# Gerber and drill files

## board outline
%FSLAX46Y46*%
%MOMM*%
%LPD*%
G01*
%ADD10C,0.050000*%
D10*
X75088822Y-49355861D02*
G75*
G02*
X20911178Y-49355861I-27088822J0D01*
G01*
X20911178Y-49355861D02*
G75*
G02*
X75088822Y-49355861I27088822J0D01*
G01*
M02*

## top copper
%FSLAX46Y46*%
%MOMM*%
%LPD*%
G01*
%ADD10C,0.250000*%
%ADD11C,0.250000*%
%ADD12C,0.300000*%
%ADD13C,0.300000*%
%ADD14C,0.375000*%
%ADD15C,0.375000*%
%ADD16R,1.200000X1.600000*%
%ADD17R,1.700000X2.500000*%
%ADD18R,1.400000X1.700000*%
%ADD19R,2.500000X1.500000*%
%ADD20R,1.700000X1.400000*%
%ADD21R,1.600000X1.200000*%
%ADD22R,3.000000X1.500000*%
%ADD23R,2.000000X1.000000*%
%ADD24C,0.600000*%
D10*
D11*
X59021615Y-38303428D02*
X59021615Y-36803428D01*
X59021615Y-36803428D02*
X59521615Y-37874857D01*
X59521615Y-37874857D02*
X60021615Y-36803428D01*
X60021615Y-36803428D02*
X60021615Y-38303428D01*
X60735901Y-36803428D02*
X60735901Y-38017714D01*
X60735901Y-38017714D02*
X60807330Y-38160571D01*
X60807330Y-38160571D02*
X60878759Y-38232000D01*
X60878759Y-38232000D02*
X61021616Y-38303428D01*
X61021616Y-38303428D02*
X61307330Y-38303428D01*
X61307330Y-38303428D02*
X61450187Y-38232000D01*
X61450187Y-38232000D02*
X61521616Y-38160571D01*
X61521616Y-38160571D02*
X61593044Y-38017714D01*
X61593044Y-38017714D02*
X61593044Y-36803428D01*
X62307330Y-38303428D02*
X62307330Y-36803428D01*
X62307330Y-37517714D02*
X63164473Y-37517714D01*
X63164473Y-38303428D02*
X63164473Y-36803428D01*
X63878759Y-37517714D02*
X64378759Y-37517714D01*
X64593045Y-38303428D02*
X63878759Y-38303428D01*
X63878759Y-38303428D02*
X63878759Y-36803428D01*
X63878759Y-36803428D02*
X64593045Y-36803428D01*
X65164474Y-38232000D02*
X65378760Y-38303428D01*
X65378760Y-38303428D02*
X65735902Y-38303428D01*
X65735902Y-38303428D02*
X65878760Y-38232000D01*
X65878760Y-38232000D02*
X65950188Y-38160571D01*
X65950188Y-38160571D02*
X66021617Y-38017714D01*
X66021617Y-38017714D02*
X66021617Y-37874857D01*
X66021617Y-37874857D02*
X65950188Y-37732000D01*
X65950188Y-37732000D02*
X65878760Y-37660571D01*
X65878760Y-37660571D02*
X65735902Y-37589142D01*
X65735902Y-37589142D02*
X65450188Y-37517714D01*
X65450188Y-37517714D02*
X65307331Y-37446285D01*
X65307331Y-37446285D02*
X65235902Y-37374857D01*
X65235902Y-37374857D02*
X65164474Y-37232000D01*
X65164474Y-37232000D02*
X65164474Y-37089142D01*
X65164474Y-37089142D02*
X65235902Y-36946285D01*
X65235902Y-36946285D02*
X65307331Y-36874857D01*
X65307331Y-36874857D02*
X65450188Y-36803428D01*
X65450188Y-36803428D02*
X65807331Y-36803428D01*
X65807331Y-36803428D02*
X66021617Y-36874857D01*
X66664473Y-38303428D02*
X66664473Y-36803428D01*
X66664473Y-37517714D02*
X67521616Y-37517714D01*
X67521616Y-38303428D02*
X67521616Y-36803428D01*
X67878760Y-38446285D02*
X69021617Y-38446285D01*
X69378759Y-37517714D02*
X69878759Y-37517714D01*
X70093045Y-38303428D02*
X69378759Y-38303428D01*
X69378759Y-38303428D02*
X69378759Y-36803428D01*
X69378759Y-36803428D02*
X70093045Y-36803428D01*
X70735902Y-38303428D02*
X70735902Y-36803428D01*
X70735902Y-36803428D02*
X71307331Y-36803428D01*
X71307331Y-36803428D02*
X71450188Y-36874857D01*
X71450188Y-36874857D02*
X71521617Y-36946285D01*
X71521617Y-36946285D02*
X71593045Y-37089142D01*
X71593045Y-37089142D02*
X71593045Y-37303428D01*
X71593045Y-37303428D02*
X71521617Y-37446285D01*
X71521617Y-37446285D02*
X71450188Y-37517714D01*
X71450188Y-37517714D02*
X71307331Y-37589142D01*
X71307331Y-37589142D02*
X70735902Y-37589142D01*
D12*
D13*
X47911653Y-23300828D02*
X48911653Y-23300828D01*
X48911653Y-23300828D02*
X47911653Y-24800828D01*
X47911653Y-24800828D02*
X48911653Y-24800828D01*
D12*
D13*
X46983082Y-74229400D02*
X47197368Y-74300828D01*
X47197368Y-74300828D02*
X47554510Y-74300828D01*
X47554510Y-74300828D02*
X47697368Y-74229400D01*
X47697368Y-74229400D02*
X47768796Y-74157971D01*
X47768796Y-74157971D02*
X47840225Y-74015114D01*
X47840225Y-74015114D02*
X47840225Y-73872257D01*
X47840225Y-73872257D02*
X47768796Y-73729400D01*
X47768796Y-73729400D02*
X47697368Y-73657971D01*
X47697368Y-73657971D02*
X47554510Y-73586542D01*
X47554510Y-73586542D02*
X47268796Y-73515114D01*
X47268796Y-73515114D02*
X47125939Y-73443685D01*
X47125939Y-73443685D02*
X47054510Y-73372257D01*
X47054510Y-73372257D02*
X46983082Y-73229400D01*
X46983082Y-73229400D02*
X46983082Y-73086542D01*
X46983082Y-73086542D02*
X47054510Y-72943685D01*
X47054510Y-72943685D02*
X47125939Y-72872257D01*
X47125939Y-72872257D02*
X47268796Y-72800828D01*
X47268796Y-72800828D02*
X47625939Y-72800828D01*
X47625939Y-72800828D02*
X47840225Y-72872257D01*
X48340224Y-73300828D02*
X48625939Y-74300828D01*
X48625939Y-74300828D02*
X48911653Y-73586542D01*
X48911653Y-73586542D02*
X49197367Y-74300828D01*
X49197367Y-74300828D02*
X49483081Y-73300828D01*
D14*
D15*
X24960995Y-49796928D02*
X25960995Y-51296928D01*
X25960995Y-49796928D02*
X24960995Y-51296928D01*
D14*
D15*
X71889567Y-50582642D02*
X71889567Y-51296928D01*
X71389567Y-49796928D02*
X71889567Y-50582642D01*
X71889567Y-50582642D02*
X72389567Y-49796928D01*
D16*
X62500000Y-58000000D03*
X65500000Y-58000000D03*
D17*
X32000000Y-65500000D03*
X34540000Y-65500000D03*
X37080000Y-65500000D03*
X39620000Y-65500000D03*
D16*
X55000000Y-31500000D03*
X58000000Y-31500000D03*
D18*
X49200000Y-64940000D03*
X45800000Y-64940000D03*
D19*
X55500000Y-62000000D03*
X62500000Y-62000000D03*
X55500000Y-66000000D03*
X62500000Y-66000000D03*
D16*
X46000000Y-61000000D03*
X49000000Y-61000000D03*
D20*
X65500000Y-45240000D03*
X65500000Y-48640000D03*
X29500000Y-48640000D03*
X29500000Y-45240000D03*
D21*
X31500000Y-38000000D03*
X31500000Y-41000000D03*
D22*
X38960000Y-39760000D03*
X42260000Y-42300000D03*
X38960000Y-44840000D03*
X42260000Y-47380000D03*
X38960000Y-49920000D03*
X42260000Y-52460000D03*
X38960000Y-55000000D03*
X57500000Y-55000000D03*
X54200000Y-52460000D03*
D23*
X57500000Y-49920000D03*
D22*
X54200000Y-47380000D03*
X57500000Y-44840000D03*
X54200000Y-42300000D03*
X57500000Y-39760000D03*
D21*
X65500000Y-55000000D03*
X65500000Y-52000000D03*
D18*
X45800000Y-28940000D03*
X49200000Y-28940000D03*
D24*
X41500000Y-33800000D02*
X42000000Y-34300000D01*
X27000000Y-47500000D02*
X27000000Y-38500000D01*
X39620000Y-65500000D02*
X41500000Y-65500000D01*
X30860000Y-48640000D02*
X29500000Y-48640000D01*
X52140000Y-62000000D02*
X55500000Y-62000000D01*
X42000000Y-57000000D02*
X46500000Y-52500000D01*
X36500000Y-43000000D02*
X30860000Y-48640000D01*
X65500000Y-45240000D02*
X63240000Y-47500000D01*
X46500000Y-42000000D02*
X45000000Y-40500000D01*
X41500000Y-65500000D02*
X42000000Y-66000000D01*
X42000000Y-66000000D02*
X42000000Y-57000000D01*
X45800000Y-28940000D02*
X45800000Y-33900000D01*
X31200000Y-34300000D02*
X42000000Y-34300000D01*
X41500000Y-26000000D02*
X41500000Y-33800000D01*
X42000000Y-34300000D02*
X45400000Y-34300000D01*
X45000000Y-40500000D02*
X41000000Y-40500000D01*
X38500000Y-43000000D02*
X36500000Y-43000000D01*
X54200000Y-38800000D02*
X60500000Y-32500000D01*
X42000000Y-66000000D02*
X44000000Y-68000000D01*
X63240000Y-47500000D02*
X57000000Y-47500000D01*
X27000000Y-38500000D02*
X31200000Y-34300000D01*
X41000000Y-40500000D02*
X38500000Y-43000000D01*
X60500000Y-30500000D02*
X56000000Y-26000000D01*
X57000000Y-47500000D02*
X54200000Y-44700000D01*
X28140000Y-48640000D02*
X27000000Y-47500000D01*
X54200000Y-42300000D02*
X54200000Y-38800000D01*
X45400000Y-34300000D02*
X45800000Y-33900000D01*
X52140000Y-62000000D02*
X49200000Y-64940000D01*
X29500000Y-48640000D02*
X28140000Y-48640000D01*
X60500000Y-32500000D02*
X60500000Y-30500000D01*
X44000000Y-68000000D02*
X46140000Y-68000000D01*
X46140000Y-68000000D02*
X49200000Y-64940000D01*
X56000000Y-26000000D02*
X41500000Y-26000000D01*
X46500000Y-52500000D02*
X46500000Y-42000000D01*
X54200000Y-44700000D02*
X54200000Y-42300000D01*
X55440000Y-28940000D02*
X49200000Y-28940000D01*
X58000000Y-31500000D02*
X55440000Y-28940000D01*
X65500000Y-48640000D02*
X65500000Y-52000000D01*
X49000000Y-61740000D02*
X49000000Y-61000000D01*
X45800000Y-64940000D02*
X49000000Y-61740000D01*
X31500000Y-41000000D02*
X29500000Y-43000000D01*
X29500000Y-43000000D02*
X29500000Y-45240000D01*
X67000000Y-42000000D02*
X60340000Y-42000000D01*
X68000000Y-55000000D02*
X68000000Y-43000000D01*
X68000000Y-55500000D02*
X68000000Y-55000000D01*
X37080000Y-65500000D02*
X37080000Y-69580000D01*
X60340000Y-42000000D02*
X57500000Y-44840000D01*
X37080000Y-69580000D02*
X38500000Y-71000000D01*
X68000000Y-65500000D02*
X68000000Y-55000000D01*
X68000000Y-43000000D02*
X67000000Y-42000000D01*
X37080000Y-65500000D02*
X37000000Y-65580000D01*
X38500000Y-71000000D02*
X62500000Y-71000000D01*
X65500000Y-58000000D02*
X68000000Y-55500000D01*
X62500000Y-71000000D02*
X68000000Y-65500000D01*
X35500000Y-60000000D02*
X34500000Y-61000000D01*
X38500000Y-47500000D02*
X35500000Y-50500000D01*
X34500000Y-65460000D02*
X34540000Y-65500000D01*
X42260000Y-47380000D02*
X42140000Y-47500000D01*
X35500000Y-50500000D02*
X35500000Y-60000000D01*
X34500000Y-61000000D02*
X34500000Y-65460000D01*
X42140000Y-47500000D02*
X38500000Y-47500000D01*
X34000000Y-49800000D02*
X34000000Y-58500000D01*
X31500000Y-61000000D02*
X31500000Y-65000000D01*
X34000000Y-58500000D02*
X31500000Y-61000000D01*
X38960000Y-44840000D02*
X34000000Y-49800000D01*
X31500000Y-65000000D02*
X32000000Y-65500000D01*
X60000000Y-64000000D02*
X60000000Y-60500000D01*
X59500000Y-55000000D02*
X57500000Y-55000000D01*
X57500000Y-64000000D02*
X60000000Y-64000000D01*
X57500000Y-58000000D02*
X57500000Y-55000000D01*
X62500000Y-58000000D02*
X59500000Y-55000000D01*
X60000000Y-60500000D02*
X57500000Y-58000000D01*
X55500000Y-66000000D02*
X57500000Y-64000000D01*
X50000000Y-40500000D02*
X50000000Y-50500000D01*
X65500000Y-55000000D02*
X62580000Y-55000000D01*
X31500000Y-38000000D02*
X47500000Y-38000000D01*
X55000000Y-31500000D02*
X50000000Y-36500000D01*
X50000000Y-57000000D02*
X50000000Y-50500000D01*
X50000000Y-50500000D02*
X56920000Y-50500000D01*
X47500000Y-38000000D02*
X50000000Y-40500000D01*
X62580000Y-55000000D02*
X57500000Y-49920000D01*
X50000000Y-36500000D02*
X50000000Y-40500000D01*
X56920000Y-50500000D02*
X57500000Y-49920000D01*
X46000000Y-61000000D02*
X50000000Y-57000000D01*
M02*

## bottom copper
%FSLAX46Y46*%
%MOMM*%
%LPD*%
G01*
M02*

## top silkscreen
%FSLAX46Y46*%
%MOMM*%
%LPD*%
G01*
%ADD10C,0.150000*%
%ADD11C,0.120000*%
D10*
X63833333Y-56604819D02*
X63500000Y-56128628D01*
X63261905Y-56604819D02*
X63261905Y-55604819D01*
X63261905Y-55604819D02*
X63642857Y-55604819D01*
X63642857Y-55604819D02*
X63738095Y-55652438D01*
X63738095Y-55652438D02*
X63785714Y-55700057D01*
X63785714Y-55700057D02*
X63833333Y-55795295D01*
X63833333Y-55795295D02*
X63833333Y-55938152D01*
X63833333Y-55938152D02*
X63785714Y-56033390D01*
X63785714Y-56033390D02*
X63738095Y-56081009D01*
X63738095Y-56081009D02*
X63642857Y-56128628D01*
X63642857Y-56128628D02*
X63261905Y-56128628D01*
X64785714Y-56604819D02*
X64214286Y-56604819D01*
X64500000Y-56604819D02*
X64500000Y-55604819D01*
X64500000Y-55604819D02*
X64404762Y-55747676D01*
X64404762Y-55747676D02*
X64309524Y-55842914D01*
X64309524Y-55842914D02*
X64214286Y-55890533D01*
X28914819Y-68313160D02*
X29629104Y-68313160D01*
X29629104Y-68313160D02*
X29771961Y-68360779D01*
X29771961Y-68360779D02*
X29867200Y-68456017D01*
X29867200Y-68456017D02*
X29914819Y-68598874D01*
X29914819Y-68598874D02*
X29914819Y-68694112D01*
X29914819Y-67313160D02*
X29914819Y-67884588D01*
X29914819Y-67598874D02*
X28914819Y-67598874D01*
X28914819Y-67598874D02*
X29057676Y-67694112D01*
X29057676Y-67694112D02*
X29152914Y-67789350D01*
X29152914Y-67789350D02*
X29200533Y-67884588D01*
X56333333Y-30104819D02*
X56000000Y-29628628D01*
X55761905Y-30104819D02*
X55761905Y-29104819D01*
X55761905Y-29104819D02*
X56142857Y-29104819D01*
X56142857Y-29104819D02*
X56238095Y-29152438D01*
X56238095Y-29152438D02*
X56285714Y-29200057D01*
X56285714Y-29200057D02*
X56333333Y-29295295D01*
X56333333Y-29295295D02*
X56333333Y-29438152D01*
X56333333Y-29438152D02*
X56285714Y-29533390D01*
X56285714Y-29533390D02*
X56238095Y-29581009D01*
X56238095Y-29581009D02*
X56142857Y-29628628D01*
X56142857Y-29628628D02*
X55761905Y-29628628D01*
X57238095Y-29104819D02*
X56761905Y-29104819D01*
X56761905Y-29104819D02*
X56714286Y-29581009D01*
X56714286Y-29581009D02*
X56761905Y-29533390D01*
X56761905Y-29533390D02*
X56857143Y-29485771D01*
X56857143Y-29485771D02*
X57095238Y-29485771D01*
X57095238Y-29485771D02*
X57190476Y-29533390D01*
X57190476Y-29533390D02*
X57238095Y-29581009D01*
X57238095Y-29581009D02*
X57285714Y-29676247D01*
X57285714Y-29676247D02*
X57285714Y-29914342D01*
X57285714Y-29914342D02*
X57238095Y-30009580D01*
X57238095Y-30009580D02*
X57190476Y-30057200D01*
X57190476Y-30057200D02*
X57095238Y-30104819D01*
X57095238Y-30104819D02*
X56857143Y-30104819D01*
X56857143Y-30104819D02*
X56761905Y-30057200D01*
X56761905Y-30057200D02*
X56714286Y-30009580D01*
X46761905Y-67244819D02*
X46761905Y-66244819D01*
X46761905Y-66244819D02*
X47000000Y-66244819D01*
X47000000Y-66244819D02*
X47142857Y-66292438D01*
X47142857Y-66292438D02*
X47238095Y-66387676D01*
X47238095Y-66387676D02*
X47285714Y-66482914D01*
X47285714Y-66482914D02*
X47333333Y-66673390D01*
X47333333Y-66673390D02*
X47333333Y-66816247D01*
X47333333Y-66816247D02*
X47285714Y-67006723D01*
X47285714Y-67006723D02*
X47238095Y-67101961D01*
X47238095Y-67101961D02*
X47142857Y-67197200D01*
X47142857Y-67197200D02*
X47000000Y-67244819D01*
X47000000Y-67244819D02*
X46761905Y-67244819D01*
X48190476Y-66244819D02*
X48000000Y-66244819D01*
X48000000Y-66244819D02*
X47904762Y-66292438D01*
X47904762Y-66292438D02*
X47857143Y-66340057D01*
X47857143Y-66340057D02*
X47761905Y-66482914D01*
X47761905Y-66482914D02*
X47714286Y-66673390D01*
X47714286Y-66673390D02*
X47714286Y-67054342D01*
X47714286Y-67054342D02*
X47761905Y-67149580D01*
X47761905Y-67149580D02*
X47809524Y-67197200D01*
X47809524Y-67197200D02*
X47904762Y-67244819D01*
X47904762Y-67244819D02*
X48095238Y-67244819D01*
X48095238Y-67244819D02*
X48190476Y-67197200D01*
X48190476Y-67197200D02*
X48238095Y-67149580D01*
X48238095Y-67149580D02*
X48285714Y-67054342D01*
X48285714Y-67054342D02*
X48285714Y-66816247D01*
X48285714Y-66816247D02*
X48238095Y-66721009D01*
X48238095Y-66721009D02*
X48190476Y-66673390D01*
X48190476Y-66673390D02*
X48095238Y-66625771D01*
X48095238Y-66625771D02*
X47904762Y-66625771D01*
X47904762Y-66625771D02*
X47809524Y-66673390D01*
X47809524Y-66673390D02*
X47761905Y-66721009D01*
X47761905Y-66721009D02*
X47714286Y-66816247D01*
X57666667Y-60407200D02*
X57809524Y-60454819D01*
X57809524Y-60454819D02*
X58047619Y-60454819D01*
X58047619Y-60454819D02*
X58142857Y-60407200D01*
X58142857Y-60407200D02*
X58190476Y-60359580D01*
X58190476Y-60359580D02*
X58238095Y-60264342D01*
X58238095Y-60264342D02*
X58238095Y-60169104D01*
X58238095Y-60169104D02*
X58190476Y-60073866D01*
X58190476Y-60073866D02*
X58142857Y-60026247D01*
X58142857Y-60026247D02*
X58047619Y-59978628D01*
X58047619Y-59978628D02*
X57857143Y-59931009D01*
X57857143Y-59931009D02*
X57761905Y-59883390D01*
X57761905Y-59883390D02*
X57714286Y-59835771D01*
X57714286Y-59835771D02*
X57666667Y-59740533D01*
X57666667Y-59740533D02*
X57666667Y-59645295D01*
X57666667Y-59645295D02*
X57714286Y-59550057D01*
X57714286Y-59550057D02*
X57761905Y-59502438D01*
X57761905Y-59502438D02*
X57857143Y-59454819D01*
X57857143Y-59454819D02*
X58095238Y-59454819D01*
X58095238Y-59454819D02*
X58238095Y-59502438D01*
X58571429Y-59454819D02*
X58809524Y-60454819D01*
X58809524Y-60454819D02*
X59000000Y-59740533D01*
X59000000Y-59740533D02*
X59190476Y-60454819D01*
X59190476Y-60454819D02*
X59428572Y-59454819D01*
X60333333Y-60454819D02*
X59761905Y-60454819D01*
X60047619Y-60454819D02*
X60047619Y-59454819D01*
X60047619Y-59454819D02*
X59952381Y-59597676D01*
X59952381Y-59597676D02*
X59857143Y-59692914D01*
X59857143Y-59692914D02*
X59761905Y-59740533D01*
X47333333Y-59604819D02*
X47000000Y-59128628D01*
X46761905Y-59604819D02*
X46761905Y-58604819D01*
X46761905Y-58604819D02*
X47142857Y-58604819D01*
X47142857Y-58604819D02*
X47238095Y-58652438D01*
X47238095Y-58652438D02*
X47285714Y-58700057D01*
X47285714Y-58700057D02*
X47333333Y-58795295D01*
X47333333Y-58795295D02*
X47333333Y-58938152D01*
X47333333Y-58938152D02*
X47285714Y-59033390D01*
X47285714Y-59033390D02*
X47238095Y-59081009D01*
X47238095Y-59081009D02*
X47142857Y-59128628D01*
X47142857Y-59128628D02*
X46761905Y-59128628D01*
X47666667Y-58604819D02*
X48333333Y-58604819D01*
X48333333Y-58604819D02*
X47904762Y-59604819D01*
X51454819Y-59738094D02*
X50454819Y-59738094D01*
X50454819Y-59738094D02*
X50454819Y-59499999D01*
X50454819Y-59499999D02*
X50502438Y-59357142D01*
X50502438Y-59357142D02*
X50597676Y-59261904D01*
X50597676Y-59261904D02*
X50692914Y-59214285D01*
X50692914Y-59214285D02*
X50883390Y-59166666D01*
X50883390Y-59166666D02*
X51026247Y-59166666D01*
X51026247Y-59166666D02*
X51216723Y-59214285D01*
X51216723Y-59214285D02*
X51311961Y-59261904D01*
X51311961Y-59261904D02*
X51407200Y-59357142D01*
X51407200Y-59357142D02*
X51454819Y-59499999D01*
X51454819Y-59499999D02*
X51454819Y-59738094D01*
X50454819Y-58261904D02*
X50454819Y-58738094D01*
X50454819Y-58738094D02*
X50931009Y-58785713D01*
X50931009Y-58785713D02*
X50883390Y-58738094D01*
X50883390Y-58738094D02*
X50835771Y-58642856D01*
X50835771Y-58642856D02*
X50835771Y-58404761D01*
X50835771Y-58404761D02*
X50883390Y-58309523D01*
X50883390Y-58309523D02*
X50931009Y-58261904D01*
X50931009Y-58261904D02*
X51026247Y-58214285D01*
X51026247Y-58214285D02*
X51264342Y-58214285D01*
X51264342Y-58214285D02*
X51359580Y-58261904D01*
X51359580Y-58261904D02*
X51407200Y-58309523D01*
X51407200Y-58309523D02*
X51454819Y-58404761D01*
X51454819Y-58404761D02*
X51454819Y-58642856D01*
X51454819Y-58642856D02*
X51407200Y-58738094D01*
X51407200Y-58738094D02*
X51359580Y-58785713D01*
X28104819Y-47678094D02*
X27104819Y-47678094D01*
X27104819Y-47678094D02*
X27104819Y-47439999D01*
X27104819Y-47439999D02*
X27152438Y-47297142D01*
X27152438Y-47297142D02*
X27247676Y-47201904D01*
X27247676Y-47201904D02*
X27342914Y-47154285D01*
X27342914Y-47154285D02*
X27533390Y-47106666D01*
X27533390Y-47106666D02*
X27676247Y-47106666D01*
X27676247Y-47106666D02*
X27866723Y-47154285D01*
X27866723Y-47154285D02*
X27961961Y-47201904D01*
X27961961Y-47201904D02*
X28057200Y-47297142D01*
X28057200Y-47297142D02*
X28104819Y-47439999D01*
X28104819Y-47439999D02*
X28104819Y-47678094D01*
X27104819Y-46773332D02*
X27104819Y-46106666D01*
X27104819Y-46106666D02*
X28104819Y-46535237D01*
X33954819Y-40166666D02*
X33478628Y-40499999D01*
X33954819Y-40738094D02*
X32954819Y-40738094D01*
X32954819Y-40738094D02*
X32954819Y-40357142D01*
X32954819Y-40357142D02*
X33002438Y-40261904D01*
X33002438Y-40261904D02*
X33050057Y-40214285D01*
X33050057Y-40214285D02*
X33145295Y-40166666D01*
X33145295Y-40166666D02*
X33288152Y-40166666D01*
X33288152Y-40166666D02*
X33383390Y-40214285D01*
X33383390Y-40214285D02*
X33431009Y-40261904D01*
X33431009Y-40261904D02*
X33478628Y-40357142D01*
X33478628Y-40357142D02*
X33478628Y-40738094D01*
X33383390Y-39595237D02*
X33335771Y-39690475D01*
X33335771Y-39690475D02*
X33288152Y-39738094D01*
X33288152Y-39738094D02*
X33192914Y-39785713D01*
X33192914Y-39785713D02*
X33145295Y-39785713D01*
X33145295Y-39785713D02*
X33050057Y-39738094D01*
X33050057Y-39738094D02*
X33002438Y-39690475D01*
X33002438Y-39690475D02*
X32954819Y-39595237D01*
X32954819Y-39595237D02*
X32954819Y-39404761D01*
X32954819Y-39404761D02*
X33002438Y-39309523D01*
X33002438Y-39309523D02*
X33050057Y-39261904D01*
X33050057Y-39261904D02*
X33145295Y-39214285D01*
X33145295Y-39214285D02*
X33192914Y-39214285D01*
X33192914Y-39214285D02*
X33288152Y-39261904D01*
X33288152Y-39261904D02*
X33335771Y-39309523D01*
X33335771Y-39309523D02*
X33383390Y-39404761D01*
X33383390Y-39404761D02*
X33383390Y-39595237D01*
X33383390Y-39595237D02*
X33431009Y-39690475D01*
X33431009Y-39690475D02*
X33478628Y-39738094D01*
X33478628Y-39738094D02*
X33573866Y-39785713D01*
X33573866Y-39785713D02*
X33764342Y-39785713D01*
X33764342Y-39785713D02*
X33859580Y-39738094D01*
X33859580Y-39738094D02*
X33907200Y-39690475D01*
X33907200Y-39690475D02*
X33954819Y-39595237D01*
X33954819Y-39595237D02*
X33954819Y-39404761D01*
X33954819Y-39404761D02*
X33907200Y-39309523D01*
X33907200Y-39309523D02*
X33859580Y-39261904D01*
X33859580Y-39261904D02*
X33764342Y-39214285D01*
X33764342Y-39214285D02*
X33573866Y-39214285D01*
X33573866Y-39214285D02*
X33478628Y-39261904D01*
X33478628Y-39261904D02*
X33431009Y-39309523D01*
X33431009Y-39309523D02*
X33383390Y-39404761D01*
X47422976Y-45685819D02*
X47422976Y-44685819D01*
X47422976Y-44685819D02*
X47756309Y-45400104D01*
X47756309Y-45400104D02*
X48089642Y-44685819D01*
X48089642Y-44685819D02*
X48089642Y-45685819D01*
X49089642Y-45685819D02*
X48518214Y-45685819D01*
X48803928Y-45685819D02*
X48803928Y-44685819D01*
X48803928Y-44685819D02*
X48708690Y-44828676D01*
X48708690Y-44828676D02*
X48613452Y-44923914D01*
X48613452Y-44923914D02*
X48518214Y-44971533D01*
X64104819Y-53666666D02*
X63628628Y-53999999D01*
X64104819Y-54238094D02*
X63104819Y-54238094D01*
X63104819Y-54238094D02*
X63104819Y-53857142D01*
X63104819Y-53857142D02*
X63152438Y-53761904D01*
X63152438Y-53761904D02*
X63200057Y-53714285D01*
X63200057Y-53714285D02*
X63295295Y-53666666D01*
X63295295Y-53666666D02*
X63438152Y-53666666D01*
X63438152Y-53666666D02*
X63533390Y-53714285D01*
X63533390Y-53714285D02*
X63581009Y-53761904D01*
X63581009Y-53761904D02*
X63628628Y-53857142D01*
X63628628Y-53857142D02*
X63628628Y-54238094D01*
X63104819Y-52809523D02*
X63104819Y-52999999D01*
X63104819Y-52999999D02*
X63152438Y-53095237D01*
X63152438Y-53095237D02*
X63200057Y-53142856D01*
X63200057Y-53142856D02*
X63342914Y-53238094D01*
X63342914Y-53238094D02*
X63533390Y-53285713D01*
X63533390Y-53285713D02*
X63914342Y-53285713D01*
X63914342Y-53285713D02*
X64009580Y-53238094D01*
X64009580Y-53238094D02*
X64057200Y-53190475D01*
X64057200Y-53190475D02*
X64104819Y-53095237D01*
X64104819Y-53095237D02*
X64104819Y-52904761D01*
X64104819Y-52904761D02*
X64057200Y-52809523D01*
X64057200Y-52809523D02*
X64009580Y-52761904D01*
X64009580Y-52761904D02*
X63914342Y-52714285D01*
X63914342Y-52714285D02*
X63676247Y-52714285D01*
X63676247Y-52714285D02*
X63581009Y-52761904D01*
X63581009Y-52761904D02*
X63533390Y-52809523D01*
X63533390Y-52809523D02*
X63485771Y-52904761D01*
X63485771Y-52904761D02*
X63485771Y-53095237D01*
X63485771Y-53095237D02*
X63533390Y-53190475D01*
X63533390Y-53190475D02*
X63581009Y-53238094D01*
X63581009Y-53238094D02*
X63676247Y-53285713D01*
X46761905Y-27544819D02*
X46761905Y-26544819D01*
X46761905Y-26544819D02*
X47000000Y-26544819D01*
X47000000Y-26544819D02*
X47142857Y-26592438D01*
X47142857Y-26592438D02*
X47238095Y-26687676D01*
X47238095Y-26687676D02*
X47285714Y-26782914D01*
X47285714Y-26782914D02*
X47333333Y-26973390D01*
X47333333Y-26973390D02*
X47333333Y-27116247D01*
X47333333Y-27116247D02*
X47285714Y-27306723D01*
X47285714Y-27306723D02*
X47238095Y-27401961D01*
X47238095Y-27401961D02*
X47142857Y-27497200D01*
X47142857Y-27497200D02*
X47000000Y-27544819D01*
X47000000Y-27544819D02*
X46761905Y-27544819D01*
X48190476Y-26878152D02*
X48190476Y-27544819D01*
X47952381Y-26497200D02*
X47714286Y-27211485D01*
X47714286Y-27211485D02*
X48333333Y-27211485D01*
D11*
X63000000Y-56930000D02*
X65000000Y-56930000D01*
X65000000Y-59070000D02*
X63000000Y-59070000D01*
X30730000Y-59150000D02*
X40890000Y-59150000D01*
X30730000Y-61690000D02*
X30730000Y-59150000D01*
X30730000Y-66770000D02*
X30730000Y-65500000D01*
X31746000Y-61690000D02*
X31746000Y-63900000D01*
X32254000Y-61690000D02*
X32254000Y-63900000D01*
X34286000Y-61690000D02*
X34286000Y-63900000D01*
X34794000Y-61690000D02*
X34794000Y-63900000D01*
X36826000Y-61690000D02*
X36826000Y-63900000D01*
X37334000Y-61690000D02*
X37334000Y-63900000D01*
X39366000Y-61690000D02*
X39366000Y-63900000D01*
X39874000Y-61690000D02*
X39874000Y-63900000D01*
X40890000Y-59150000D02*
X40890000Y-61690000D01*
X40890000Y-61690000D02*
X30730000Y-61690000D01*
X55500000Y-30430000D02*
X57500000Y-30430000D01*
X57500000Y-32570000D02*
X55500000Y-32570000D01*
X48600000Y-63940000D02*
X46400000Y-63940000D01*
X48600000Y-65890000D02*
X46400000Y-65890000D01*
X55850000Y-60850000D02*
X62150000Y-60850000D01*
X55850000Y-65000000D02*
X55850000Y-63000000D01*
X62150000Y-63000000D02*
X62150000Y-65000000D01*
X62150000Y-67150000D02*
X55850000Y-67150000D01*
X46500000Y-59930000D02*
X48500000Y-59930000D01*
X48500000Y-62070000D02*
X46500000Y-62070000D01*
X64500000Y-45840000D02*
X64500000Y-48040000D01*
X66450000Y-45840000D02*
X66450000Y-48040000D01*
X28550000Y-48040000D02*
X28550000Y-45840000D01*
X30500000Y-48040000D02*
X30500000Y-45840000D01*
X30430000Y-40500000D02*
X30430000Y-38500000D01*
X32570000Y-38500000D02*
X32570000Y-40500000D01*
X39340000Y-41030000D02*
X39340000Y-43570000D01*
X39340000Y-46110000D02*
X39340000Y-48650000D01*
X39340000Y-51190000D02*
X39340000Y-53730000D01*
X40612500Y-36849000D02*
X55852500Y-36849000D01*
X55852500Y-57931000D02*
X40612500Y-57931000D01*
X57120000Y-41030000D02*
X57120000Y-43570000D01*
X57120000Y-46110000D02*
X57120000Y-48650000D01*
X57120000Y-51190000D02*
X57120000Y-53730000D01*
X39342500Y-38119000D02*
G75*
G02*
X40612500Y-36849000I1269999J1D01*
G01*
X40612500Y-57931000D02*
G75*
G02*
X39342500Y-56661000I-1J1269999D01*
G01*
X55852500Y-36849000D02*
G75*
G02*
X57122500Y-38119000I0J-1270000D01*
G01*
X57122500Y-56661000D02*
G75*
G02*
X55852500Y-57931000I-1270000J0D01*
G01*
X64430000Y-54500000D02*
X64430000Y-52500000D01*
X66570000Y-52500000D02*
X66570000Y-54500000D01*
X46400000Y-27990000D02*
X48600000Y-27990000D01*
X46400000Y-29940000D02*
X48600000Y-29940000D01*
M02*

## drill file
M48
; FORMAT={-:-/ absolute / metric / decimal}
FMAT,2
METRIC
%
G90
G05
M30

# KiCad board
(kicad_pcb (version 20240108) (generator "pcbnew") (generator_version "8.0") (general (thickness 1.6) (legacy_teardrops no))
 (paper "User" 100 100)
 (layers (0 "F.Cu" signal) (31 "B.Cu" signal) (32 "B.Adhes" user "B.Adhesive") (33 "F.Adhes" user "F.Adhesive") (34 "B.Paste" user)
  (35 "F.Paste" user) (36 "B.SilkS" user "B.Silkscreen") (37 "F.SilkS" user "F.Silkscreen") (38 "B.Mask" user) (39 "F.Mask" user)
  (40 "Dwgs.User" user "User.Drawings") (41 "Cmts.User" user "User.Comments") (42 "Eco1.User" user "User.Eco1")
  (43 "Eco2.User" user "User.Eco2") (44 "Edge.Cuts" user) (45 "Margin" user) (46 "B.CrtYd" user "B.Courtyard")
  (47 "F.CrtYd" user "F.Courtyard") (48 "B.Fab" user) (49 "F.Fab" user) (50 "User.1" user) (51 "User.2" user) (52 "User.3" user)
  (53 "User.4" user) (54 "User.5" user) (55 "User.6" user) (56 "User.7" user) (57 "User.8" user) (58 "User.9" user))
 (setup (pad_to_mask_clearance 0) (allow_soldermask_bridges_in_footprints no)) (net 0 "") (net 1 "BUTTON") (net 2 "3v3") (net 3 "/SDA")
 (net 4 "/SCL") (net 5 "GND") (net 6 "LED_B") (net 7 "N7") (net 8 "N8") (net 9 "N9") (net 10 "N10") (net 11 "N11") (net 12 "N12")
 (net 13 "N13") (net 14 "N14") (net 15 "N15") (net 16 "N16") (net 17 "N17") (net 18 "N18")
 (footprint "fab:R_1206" (layer "F.Cu") (at 64 58)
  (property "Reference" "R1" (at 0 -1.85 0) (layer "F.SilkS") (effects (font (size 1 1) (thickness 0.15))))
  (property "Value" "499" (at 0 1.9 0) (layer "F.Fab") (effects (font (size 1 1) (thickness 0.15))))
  (fp_line (start -1 -1.07) (end 1 -1.07) (stroke (width 0.12) (type solid)) (layer "F.SilkS"))
  (fp_line (start 1 1.07) (end -1 1.07) (stroke (width 0.12) (type solid)) (layer "F.SilkS"))
  (pad "1" smd rect (at -1.5 0) (size 1.2 1.6) (layers "F.Cu" "F.Paste" "F.Mask") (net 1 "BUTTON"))
  (pad "2" smd rect (at 1.5 0) (size 1.2 1.6) (layers "F.Cu" "F.Paste" "F.Mask") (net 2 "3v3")))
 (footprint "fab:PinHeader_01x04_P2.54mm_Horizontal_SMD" (layer "F.Cu") (at 32 65.5 90)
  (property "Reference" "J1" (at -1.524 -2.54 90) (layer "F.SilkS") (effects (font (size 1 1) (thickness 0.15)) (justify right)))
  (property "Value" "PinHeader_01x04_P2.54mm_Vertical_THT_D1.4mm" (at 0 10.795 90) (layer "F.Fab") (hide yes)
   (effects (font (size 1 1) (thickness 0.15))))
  (fp_line (start 6.35 -1.27) (end 6.35 8.89) (stroke (width 0.12) (type solid)) (layer "F.SilkS"))
  (fp_line (start 3.81 -1.27) (end 6.35 -1.27) (stroke (width 0.12) (type solid)) (layer "F.SilkS"))
  (fp_line (start -1.27 -1.27) (end 0 -1.27) (stroke (width 0.12) (type solid)) (layer "F.SilkS"))
  (fp_line (start 3.81 -0.254) (end 1.6 -0.254) (stroke (width 0.12) (type solid)) (layer "F.SilkS"))
  (fp_line (start 3.81 0.254) (end 1.6 0.254) (stroke (width 0.12) (type solid)) (layer "F.SilkS"))
  (fp_line (start 3.81 2.286) (end 1.6 2.286) (stroke (width 0.12) (type solid)) (layer "F.SilkS"))
  (fp_line (start 3.81 2.794) (end 1.6 2.794) (stroke (width 0.12) (type solid)) (layer "F.SilkS"))
  (fp_line (start 3.81 4.826) (end 1.6 4.826) (stroke (width 0.12) (type solid)) (layer "F.SilkS"))
  (fp_line (start 3.81 5.334) (end 1.6 5.334) (stroke (width 0.12) (type solid)) (layer "F.SilkS"))
  (fp_line (start 3.81 7.366) (end 1.6 7.366) (stroke (width 0.12) (type solid)) (layer "F.SilkS"))
  (fp_line (start 3.81 7.874) (end 1.6 7.874) (stroke (width 0.12) (type solid)) (layer "F.SilkS"))
  (fp_line (start 6.35 8.89) (end 3.81 8.89) (stroke (width 0.12) (type solid)) (layer "F.SilkS"))
  (fp_line (start 3.81 8.89) (end 3.81 -1.27) (stroke (width 0.12) (type solid)) (layer "F.SilkS"))
  (pad "1" smd rect (at 0 0 90) (size 2.5 1.7) (layers "F.Cu" "F.Paste" "F.Mask") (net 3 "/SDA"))
  (pad "2" smd rect (at 0 2.54 90) (size 2.5 1.7) (layers "F.Cu" "F.Paste" "F.Mask") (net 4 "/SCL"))
  (pad "3" smd rect (at 0 5.08 90) (size 2.5 1.7) (layers "F.Cu" "F.Paste" "F.Mask") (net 2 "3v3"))
  (pad "4" smd rect (at 0 7.62 90) (size 2.5 1.7) (layers "F.Cu" "F.Paste" "F.Mask") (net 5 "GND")))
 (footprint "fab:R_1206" (layer "F.Cu") (at 56.5 31.5)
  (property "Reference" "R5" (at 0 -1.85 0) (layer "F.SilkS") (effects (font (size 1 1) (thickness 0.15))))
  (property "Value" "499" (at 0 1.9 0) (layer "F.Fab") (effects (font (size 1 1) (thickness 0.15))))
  (fp_line (start -1 -1.07) (end 1 -1.07) (stroke (width 0.12) (type solid)) (layer "F.SilkS"))
  (fp_line (start 1 1.07) (end -1 1.07) (stroke (width 0.12) (type solid)) (layer "F.SilkS"))
  (pad "1" smd rect (at -1.5 0) (size 1.2 1.6) (layers "F.Cu" "F.Paste" "F.Mask") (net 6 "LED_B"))
  (pad "2" smd rect (at 1.5 0) (size 1.2 1.6) (layers "F.Cu" "F.Paste" "F.Mask") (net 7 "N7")))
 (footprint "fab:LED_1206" (layer "F.Cu") (at 47.5 64.94 180)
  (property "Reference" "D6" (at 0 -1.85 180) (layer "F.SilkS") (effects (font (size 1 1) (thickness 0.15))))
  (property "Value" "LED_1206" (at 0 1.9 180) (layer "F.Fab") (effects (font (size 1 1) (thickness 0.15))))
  (fp_line (start -1.1 1) (end 1.1 1) (stroke (width 0.12) (type solid)) (layer "F.SilkS"))
  (fp_line (start -1.1 -0.95) (end 1.1 -0.95) (stroke (width 0.12) (type solid)) (layer "F.SilkS"))
  (pad "1" smd rect (at -1.7 0 180) (size 1.4 1.7) (layers "F.Cu" "F.Paste" "F.Mask") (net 5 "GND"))
  (pad "2" smd rect (at 1.7 0 180) (size 1.4 1.7) (layers "F.Cu" "F.Paste" "F.Mask") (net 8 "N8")))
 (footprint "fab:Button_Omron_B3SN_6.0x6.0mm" (layer "F.Cu") (at 59 64)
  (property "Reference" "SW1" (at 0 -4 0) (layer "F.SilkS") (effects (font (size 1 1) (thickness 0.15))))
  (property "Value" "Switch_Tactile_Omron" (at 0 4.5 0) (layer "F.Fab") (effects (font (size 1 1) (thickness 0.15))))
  (fp_line (start -3.15 -3.15) (end 3.15 -3.15) (stroke (width 0.12) (type solid)) (layer "F.SilkS"))
  (fp_line (start -3.15 1) (end -3.15 -1) (stroke (width 0.12) (type solid)) (layer "F.SilkS"))
  (fp_line (start 3.15 -1) (end 3.15 1) (stroke (width 0.12) (type solid)) (layer "F.SilkS"))
  (fp_line (start 3.15 3.15) (end -3.15 3.15) (stroke (width 0.12) (type solid)) (layer "F.SilkS"))
  (pad "1" smd rect (at -3.5 -2) (size 2.5 1.5) (layers "F.Cu" "F.Paste" "F.Mask") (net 5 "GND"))
  (pad "1" smd rect (at 3.5 -2) (size 2.5 1.5) (layers "F.Cu" "F.Paste" "F.Mask") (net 5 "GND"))
  (pad "2" smd rect (at -3.5 2) (size 2.5 1.5) (layers "F.Cu" "F.Paste" "F.Mask") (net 1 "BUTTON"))
  (pad "2" smd rect (at 3.5 2) (size 2.5 1.5) (layers "F.Cu" "F.Paste" "F.Mask") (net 1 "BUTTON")))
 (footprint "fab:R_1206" (layer "F.Cu") (at 47.5 61)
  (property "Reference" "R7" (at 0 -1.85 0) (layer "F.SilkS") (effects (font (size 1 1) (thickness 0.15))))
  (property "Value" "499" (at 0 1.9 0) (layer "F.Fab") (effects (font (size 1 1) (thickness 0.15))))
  (fp_line (start -1 -1.07) (end 1 -1.07) (stroke (width 0.12) (type solid)) (layer "F.SilkS"))
  (fp_line (start 1 1.07) (end -1 1.07) (stroke (width 0.12) (type solid)) (layer "F.SilkS"))
  (pad "1" smd rect (at -1.5 0) (size 1.2 1.6) (layers "F.Cu" "F.Paste" "F.Mask") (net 6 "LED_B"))
  (pad "2" smd rect (at 1.5 0) (size 1.2 1.6) (layers "F.Cu" "F.Paste" "F.Mask") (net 8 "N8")))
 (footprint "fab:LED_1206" (layer "F.Cu") (at 65.5 46.94 -90)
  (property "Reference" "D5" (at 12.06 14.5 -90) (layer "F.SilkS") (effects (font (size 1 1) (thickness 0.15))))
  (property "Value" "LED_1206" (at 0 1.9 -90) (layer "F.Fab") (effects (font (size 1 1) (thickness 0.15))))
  (fp_line (start -1.1 1) (end 1.1 1) (stroke (width 0.12) (type solid)) (layer "F.SilkS"))
  (fp_line (start -1.1 -0.95) (end 1.1 -0.95) (stroke (width 0.12) (type solid)) (layer "F.SilkS"))
  (pad "1" smd rect (at -1.7 0 270) (size 1.4 1.7) (layers "F.Cu" "F.Paste" "F.Mask") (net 5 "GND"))
  (pad "2" smd rect (at 1.7 0 270) (size 1.4 1.7) (layers "F.Cu" "F.Paste" "F.Mask") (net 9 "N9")))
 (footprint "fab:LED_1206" (layer "F.Cu") (at 29.5 46.94 90)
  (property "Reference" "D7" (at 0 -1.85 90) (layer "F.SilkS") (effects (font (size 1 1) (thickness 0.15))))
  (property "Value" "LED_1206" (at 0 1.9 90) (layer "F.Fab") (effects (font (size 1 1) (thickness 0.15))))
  (fp_line (start -1.1 -0.95) (end 1.1 -0.95) (stroke (width 0.12) (type solid)) (layer "F.SilkS"))
  (fp_line (start -1.1 1) (end 1.1 1) (stroke (width 0.12) (type solid)) (layer "F.SilkS"))
  (pad "1" smd rect (at -1.7 0 90) (size 1.4 1.7) (layers "F.Cu" "F.Paste" "F.Mask") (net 5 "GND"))
  (pad "2" smd rect (at 1.7 0 90) (size 1.4 1.7) (layers "F.Cu" "F.Paste" "F.Mask") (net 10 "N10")))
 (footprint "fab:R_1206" (layer "F.Cu") (at 31.5 39.5 -90)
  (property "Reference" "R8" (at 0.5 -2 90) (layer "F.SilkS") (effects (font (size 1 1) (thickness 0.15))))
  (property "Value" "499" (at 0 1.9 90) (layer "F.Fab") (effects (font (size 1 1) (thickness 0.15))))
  (fp_line (start 1 1.07) (end -1 1.07) (stroke (width 0.12) (type solid)) (layer "F.SilkS"))
  (fp_line (start -1 -1.07) (end 1 -1.07) (stroke (width 0.12) (type solid)) (layer "F.SilkS"))
  (pad "1" smd rect (at -1.5 0 270) (size 1.2 1.6) (layers "F.Cu" "F.Paste" "F.Mask") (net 6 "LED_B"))
  (pad "2" smd rect (at 1.5 0 270) (size 1.2 1.6) (layers "F.Cu" "F.Paste" "F.Mask") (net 10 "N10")))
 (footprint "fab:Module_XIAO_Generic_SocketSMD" (layer "F.Cu") (at 48.23 47.38)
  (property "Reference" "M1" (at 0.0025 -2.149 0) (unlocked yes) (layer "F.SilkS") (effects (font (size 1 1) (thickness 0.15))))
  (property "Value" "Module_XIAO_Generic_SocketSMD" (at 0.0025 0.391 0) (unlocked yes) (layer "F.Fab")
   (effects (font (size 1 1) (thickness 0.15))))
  (fp_line (start -8.89 -6.35) (end -8.89 -3.81) (stroke (width 0.12) (type default)) (layer "F.SilkS"))
  (fp_line (start -8.89 -1.27) (end -8.89 1.27) (stroke (width 0.12) (type default)) (layer "F.SilkS"))
  (fp_line (start -8.89 3.81) (end -8.89 6.35) (stroke (width 0.12) (type default)) (layer "F.SilkS"))
  (fp_line (start -7.6175 -10.531) (end 7.6225 -10.531) (stroke (width 0.12) (type solid)) (layer "F.SilkS"))
  (fp_line (start 7.6225 10.551) (end -7.6175 10.551) (stroke (width 0.12) (type solid)) (layer "F.SilkS"))
  (fp_line (start 8.89 -6.35) (end 8.89 -3.81) (stroke (width 0.12) (type default)) (layer "F.SilkS"))
  (fp_line (start 8.89 -1.27) (end 8.89 1.27) (stroke (width 0.12) (type default)) (layer "F.SilkS"))
  (fp_line (start 8.89 3.81) (end 8.89 6.35) (stroke (width 0.12) (type default)) (layer "F.SilkS"))
  (fp_arc (start -8.8875 -9.261) (mid -8.515526 -10.159026) (end -7.6175 -10.531) (stroke (width 0.12) (type solid)) (layer "F.SilkS"))
  (fp_arc (start -7.6175 10.551) (mid -8.515526 10.179026) (end -8.8875 9.281) (stroke (width 0.12) (type solid)) (layer "F.SilkS"))
  (fp_arc (start 7.6225 -10.531) (mid 8.520526 -10.159026) (end 8.8925 -9.261) (stroke (width 0.12) (type solid)) (layer "F.SilkS"))
  (fp_arc (start 8.8925 9.281) (mid 8.520526 10.179026) (end 7.6225 10.551) (stroke (width 0.12) (type solid)) (layer "F.SilkS"))
  (pad "1" smd rect (at -9.27 -7.62) (size 3 1.5) (layers "F.Cu" "F.Paste" "F.Mask") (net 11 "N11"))
  (pad "2" smd rect (at -5.97 -5.08) (size 3 1.5) (layers "F.Cu" "F.Paste" "F.Mask") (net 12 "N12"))
  (pad "3" smd rect (at -9.27 -2.54) (size 3 1.5) (layers "F.Cu" "F.Paste" "F.Mask") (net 3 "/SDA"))
  (pad "4" smd rect (at -5.97 0) (size 3 1.5) (layers "F.Cu" "F.Paste" "F.Mask") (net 4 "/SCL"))
  (pad "5" smd rect (at -9.27 2.54) (size 3 1.5) (layers "F.Cu" "F.Paste" "F.Mask") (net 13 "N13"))
  (pad "6" smd rect (at -5.97 5.08) (size 3 1.5) (layers "F.Cu" "F.Paste" "F.Mask") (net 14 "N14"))
  (pad "7" smd rect (at -9.27 7.62) (size 3 1.5) (layers "F.Cu" "F.Paste" "F.Mask") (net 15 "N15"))
  (pad "8" smd rect (at 9.27 7.62) (size 3 1.5) (layers "F.Cu" "F.Paste" "F.Mask") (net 1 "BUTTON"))
  (pad "9" smd rect (at 5.97 5.08) (size 3 1.5) (layers "F.Cu" "F.Paste" "F.Mask") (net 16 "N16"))
  (pad "10" smd rect (at 9.27 2.54) (size 2 1) (layers "F.Cu" "F.Paste" "F.Mask") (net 6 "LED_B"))
  (pad "11" smd rect (at 5.97 0) (size 3 1.5) (layers "F.Cu" "F.Paste" "F.Mask") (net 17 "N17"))
  (pad "12" smd rect (at 9.27 -2.54) (size 3 1.5) (layers "F.Cu" "F.Paste" "F.Mask") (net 2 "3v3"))
  (pad "13" smd rect (at 5.97 -5.08) (size 3 1.5) (layers "F.Cu" "F.Paste" "F.Mask") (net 5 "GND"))
  (pad "14" smd rect (at 9.27 -7.62) (size 3 1.5) (layers "F.Cu" "F.Paste" "F.Mask") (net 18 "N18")))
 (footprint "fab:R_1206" (layer "F.Cu") (at 65.5 53.5 90)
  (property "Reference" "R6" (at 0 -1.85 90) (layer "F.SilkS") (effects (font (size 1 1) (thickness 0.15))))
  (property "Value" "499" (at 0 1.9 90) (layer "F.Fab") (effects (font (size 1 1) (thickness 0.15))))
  (fp_line (start -1 -1.07) (end 1 -1.07) (stroke (width 0.12) (type solid)) (layer "F.SilkS"))
  (fp_line (start 1 1.07) (end -1 1.07) (stroke (width 0.12) (type solid)) (layer "F.SilkS"))
  (pad "1" smd rect (at -1.5 0 90) (size 1.2 1.6) (layers "F.Cu" "F.Paste" "F.Mask") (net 6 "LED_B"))
  (pad "2" smd rect (at 1.5 0 90) (size 1.2 1.6) (layers "F.Cu" "F.Paste" "F.Mask") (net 9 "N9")))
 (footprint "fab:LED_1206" (layer "F.Cu") (at 47.5 28.94)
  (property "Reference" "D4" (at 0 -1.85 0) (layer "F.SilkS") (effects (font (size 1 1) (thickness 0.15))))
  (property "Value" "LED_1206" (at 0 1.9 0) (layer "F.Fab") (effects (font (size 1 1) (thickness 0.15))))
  (fp_line (start -1.1 -0.95) (end 1.1 -0.95) (stroke (width 0.12) (type solid)) (layer "F.SilkS"))
  (fp_line (start -1.1 1) (end 1.1 1) (stroke (width 0.12) (type solid)) (layer "F.SilkS"))
  (pad "1" smd rect (at -1.7 0) (size 1.4 1.7) (layers "F.Cu" "F.Paste" "F.Mask") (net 5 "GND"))
  (pad "2" smd rect (at 1.7 0) (size 1.4 1.7) (layers "F.Cu" "F.Paste" "F.Mask") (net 7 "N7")))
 (gr_circle (center 48 49.355861) (end 47 76.426219) (stroke (width 0.05) (type default)) (fill none) (layer "Edge.Cuts"))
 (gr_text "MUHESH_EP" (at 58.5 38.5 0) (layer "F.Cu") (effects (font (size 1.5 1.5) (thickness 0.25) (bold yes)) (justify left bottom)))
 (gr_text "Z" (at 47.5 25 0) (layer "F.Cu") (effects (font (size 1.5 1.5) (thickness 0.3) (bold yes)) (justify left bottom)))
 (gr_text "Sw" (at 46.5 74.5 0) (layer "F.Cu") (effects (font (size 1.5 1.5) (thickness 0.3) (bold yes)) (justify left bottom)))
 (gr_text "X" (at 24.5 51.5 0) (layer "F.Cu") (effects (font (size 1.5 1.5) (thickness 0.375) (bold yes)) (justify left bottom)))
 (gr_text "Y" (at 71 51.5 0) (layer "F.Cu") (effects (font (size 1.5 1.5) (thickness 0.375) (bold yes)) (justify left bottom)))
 (segment (start 41.5 33.8) (end 42 34.3) (width 0.6) (layer "F.Cu") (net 5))
 (segment (start 27 47.5) (end 27 38.5) (width 0.6) (layer "F.Cu") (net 5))
 (segment (start 39.62 65.5) (end 41.5 65.5) (width 0.6) (layer "F.Cu") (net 5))
 (segment (start 30.86 48.64) (end 29.5 48.64) (width 0.6) (layer "F.Cu") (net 5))
 (segment (start 52.14 62) (end 55.5 62) (width 0.6) (layer "F.Cu") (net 5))
 (segment (start 42 57) (end 46.5 52.5) (width 0.6) (layer "F.Cu") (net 5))
 (segment (start 36.5 43) (end 30.86 48.64) (width 0.6) (layer "F.Cu") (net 5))
 (segment (start 65.5 45.24) (end 63.24 47.5) (width 0.6) (layer "F.Cu") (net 5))
 (segment (start 46.5 42) (end 45 40.5) (width 0.6) (layer "F.Cu") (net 5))
 (segment (start 41.5 65.5) (end 42 66) (width 0.6) (layer "F.Cu") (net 5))
 (segment (start 42 66) (end 42 57) (width 0.6) (layer "F.Cu") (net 5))
 (segment (start 45.8 28.94) (end 45.8 33.9) (width 0.6) (layer "F.Cu") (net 5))
 (segment (start 31.2 34.3) (end 42 34.3) (width 0.6) (layer "F.Cu") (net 5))
 (segment (start 41.5 26) (end 41.5 33.8) (width 0.6) (layer "F.Cu") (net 5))
 (segment (start 42 34.3) (end 45.4 34.3) (width 0.6) (layer "F.Cu") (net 5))
 (segment (start 45 40.5) (end 41 40.5) (width 0.6) (layer "F.Cu") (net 5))
 (segment (start 38.5 43) (end 36.5 43) (width 0.6) (layer "F.Cu") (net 5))
 (segment (start 54.2 38.8) (end 60.5 32.5) (width 0.6) (layer "F.Cu") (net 5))
 (segment (start 42 66) (end 44 68) (width 0.6) (layer "F.Cu") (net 5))
 (segment (start 63.24 47.5) (end 57 47.5) (width 0.6) (layer "F.Cu") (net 5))
 (segment (start 27 38.5) (end 31.2 34.3) (width 0.6) (layer "F.Cu") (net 5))
 (segment (start 41 40.5) (end 38.5 43) (width 0.6) (layer "F.Cu") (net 5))
 (segment (start 60.5 30.5) (end 56 26) (width 0.6) (layer "F.Cu") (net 5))
 (segment (start 57 47.5) (end 54.2 44.7) (width 0.6) (layer "F.Cu") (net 5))
 (segment (start 28.14 48.64) (end 27 47.5) (width 0.6) (layer "F.Cu") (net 5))
 (segment (start 54.2 42.3) (end 54.2 38.8) (width 0.6) (layer "F.Cu") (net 5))
 (segment (start 45.4 34.3) (end 45.8 33.9) (width 0.6) (layer "F.Cu") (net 5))
 (segment (start 52.14 62) (end 49.2 64.94) (width 0.6) (layer "F.Cu") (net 5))
 (segment (start 29.5 48.64) (end 28.14 48.64) (width 0.6) (layer "F.Cu") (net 5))
 (segment (start 60.5 32.5) (end 60.5 30.5) (width 0.6) (layer "F.Cu") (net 5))
 (segment (start 44 68) (end 46.14 68) (width 0.6) (layer "F.Cu") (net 5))
 (segment (start 46.14 68) (end 49.2 64.94) (width 0.6) (layer "F.Cu") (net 5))
 (segment (start 56 26) (end 41.5 26) (width 0.6) (layer "F.Cu") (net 5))
 (segment (start 46.5 52.5) (end 46.5 42) (width 0.6) (layer "F.Cu") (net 5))
 (segment (start 54.2 44.7) (end 54.2 42.3) (width 0.6) (layer "F.Cu") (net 5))
 (segment (start 55.44 28.94) (end 49.2 28.94) (width 0.6) (layer "F.Cu") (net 7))
 (segment (start 58 31.5) (end 55.44 28.94) (width 0.6) (layer "F.Cu") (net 7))
 (segment (start 65.5 48.64) (end 65.5 52) (width 0.6) (layer "F.Cu") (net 9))
 (segment (start 49 61.74) (end 49 61) (width 0.6) (layer "F.Cu") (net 8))
 (segment (start 45.8 64.94) (end 49 61.74) (width 0.6) (layer "F.Cu") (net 8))
 (segment (start 31.5 41) (end 29.5 43) (width 0.6) (layer "F.Cu") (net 10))
 (segment (start 29.5 43) (end 29.5 45.24) (width 0.6) (layer "F.Cu") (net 10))
 (segment (start 67 42) (end 60.34 42) (width 0.6) (layer "F.Cu") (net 2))
 (segment (start 68 55) (end 68 43) (width 0.6) (layer "F.Cu") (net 2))
 (segment (start 68 55.5) (end 68 55) (width 0.6) (layer "F.Cu") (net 2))
 (segment (start 37.08 65.5) (end 37.08 69.58) (width 0.6) (layer "F.Cu") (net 2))
 (segment (start 60.34 42) (end 57.5 44.84) (width 0.6) (layer "F.Cu") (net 2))
 (segment (start 37.08 69.58) (end 38.5 71) (width 0.6) (layer "F.Cu") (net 2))
 (segment (start 68 65.5) (end 68 55) (width 0.6) (layer "F.Cu") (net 2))
 (segment (start 68 43) (end 67 42) (width 0.6) (layer "F.Cu") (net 2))
 (segment (start 37.08 65.5) (end 37 65.58) (width 0.6) (layer "F.Cu") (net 2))
 (segment (start 38.5 71) (end 62.5 71) (width 0.6) (layer "F.Cu") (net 2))
 (segment (start 65.5 58) (end 68 55.5) (width 0.6) (layer "F.Cu") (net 2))
 (segment (start 62.5 71) (end 68 65.5) (width 0.6) (layer "F.Cu") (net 2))
 (segment (start 35.5 60) (end 34.5 61) (width 0.6) (layer "F.Cu") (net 4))
 (segment (start 38.5 47.5) (end 35.5 50.5) (width 0.6) (layer "F.Cu") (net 4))
 (segment (start 34.5 65.46) (end 34.54 65.5) (width 0.6) (layer "F.Cu") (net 4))
 (segment (start 42.26 47.38) (end 42.14 47.5) (width 0.6) (layer "F.Cu") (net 4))
 (segment (start 35.5 50.5) (end 35.5 60) (width 0.6) (layer "F.Cu") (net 4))
 (segment (start 34.5 61) (end 34.5 65.46) (width 0.6) (layer "F.Cu") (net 4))
 (segment (start 42.14 47.5) (end 38.5 47.5) (width 0.6) (layer "F.Cu") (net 4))
 (segment (start 34 49.8) (end 34 58.5) (width 0.6) (layer "F.Cu") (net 3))
 (segment (start 31.5 61) (end 31.5 65) (width 0.6) (layer "F.Cu") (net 3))
 (segment (start 34 58.5) (end 31.5 61) (width 0.6) (layer "F.Cu") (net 3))
 (segment (start 38.96 44.84) (end 34 49.8) (width 0.6) (layer "F.Cu") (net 3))
 (segment (start 31.5 65) (end 32 65.5) (width 0.6) (layer "F.Cu") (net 3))
 (segment (start 60 64) (end 60 60.5) (width 0.6) (layer "F.Cu") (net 1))
 (segment (start 59.5 55) (end 57.5 55) (width 0.6) (layer "F.Cu") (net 1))
 (segment (start 57.5 64) (end 60 64) (width 0.6) (layer "F.Cu") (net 1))
 (segment (start 57.5 58) (end 57.5 55) (width 0.6) (layer "F.Cu") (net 1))
 (segment (start 62.5 58) (end 59.5 55) (width 0.6) (layer "F.Cu") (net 1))
 (segment (start 60 60.5) (end 57.5 58) (width 0.6) (layer "F.Cu") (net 1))
 (segment (start 55.5 66) (end 57.5 64) (width 0.6) (layer "F.Cu") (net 1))
 (segment (start 50 40.5) (end 50 50.5) (width 0.6) (layer "F.Cu") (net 6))
 (segment (start 65.5 55) (end 62.58 55) (width 0.6) (layer "F.Cu") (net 6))
 (segment (start 31.5 38) (end 47.5 38) (width 0.6) (layer "F.Cu") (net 6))
 (segment (start 55 31.5) (end 50 36.5) (width 0.6) (layer "F.Cu") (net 6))
 (segment (start 50 57) (end 50 50.5) (width 0.6) (layer "F.Cu") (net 6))
 (segment (start 50 50.5) (end 56.92 50.5) (width 0.6) (layer "F.Cu") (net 6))
 (segment (start 47.5 38) (end 50 40.5) (width 0.6) (layer "F.Cu") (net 6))
 (segment (start 62.58 55) (end 57.5 49.92) (width 0.6) (layer "F.Cu") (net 6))
 (segment (start 50 36.5) (end 50 40.5) (width 0.6) (layer "F.Cu") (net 6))
 (segment (start 56.92 50.5) (end 57.5 49.92) (width 0.6) (layer "F.Cu") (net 6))
 (segment (start 46 61) (end 50 57) (width 0.6) (layer "F.Cu") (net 6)))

